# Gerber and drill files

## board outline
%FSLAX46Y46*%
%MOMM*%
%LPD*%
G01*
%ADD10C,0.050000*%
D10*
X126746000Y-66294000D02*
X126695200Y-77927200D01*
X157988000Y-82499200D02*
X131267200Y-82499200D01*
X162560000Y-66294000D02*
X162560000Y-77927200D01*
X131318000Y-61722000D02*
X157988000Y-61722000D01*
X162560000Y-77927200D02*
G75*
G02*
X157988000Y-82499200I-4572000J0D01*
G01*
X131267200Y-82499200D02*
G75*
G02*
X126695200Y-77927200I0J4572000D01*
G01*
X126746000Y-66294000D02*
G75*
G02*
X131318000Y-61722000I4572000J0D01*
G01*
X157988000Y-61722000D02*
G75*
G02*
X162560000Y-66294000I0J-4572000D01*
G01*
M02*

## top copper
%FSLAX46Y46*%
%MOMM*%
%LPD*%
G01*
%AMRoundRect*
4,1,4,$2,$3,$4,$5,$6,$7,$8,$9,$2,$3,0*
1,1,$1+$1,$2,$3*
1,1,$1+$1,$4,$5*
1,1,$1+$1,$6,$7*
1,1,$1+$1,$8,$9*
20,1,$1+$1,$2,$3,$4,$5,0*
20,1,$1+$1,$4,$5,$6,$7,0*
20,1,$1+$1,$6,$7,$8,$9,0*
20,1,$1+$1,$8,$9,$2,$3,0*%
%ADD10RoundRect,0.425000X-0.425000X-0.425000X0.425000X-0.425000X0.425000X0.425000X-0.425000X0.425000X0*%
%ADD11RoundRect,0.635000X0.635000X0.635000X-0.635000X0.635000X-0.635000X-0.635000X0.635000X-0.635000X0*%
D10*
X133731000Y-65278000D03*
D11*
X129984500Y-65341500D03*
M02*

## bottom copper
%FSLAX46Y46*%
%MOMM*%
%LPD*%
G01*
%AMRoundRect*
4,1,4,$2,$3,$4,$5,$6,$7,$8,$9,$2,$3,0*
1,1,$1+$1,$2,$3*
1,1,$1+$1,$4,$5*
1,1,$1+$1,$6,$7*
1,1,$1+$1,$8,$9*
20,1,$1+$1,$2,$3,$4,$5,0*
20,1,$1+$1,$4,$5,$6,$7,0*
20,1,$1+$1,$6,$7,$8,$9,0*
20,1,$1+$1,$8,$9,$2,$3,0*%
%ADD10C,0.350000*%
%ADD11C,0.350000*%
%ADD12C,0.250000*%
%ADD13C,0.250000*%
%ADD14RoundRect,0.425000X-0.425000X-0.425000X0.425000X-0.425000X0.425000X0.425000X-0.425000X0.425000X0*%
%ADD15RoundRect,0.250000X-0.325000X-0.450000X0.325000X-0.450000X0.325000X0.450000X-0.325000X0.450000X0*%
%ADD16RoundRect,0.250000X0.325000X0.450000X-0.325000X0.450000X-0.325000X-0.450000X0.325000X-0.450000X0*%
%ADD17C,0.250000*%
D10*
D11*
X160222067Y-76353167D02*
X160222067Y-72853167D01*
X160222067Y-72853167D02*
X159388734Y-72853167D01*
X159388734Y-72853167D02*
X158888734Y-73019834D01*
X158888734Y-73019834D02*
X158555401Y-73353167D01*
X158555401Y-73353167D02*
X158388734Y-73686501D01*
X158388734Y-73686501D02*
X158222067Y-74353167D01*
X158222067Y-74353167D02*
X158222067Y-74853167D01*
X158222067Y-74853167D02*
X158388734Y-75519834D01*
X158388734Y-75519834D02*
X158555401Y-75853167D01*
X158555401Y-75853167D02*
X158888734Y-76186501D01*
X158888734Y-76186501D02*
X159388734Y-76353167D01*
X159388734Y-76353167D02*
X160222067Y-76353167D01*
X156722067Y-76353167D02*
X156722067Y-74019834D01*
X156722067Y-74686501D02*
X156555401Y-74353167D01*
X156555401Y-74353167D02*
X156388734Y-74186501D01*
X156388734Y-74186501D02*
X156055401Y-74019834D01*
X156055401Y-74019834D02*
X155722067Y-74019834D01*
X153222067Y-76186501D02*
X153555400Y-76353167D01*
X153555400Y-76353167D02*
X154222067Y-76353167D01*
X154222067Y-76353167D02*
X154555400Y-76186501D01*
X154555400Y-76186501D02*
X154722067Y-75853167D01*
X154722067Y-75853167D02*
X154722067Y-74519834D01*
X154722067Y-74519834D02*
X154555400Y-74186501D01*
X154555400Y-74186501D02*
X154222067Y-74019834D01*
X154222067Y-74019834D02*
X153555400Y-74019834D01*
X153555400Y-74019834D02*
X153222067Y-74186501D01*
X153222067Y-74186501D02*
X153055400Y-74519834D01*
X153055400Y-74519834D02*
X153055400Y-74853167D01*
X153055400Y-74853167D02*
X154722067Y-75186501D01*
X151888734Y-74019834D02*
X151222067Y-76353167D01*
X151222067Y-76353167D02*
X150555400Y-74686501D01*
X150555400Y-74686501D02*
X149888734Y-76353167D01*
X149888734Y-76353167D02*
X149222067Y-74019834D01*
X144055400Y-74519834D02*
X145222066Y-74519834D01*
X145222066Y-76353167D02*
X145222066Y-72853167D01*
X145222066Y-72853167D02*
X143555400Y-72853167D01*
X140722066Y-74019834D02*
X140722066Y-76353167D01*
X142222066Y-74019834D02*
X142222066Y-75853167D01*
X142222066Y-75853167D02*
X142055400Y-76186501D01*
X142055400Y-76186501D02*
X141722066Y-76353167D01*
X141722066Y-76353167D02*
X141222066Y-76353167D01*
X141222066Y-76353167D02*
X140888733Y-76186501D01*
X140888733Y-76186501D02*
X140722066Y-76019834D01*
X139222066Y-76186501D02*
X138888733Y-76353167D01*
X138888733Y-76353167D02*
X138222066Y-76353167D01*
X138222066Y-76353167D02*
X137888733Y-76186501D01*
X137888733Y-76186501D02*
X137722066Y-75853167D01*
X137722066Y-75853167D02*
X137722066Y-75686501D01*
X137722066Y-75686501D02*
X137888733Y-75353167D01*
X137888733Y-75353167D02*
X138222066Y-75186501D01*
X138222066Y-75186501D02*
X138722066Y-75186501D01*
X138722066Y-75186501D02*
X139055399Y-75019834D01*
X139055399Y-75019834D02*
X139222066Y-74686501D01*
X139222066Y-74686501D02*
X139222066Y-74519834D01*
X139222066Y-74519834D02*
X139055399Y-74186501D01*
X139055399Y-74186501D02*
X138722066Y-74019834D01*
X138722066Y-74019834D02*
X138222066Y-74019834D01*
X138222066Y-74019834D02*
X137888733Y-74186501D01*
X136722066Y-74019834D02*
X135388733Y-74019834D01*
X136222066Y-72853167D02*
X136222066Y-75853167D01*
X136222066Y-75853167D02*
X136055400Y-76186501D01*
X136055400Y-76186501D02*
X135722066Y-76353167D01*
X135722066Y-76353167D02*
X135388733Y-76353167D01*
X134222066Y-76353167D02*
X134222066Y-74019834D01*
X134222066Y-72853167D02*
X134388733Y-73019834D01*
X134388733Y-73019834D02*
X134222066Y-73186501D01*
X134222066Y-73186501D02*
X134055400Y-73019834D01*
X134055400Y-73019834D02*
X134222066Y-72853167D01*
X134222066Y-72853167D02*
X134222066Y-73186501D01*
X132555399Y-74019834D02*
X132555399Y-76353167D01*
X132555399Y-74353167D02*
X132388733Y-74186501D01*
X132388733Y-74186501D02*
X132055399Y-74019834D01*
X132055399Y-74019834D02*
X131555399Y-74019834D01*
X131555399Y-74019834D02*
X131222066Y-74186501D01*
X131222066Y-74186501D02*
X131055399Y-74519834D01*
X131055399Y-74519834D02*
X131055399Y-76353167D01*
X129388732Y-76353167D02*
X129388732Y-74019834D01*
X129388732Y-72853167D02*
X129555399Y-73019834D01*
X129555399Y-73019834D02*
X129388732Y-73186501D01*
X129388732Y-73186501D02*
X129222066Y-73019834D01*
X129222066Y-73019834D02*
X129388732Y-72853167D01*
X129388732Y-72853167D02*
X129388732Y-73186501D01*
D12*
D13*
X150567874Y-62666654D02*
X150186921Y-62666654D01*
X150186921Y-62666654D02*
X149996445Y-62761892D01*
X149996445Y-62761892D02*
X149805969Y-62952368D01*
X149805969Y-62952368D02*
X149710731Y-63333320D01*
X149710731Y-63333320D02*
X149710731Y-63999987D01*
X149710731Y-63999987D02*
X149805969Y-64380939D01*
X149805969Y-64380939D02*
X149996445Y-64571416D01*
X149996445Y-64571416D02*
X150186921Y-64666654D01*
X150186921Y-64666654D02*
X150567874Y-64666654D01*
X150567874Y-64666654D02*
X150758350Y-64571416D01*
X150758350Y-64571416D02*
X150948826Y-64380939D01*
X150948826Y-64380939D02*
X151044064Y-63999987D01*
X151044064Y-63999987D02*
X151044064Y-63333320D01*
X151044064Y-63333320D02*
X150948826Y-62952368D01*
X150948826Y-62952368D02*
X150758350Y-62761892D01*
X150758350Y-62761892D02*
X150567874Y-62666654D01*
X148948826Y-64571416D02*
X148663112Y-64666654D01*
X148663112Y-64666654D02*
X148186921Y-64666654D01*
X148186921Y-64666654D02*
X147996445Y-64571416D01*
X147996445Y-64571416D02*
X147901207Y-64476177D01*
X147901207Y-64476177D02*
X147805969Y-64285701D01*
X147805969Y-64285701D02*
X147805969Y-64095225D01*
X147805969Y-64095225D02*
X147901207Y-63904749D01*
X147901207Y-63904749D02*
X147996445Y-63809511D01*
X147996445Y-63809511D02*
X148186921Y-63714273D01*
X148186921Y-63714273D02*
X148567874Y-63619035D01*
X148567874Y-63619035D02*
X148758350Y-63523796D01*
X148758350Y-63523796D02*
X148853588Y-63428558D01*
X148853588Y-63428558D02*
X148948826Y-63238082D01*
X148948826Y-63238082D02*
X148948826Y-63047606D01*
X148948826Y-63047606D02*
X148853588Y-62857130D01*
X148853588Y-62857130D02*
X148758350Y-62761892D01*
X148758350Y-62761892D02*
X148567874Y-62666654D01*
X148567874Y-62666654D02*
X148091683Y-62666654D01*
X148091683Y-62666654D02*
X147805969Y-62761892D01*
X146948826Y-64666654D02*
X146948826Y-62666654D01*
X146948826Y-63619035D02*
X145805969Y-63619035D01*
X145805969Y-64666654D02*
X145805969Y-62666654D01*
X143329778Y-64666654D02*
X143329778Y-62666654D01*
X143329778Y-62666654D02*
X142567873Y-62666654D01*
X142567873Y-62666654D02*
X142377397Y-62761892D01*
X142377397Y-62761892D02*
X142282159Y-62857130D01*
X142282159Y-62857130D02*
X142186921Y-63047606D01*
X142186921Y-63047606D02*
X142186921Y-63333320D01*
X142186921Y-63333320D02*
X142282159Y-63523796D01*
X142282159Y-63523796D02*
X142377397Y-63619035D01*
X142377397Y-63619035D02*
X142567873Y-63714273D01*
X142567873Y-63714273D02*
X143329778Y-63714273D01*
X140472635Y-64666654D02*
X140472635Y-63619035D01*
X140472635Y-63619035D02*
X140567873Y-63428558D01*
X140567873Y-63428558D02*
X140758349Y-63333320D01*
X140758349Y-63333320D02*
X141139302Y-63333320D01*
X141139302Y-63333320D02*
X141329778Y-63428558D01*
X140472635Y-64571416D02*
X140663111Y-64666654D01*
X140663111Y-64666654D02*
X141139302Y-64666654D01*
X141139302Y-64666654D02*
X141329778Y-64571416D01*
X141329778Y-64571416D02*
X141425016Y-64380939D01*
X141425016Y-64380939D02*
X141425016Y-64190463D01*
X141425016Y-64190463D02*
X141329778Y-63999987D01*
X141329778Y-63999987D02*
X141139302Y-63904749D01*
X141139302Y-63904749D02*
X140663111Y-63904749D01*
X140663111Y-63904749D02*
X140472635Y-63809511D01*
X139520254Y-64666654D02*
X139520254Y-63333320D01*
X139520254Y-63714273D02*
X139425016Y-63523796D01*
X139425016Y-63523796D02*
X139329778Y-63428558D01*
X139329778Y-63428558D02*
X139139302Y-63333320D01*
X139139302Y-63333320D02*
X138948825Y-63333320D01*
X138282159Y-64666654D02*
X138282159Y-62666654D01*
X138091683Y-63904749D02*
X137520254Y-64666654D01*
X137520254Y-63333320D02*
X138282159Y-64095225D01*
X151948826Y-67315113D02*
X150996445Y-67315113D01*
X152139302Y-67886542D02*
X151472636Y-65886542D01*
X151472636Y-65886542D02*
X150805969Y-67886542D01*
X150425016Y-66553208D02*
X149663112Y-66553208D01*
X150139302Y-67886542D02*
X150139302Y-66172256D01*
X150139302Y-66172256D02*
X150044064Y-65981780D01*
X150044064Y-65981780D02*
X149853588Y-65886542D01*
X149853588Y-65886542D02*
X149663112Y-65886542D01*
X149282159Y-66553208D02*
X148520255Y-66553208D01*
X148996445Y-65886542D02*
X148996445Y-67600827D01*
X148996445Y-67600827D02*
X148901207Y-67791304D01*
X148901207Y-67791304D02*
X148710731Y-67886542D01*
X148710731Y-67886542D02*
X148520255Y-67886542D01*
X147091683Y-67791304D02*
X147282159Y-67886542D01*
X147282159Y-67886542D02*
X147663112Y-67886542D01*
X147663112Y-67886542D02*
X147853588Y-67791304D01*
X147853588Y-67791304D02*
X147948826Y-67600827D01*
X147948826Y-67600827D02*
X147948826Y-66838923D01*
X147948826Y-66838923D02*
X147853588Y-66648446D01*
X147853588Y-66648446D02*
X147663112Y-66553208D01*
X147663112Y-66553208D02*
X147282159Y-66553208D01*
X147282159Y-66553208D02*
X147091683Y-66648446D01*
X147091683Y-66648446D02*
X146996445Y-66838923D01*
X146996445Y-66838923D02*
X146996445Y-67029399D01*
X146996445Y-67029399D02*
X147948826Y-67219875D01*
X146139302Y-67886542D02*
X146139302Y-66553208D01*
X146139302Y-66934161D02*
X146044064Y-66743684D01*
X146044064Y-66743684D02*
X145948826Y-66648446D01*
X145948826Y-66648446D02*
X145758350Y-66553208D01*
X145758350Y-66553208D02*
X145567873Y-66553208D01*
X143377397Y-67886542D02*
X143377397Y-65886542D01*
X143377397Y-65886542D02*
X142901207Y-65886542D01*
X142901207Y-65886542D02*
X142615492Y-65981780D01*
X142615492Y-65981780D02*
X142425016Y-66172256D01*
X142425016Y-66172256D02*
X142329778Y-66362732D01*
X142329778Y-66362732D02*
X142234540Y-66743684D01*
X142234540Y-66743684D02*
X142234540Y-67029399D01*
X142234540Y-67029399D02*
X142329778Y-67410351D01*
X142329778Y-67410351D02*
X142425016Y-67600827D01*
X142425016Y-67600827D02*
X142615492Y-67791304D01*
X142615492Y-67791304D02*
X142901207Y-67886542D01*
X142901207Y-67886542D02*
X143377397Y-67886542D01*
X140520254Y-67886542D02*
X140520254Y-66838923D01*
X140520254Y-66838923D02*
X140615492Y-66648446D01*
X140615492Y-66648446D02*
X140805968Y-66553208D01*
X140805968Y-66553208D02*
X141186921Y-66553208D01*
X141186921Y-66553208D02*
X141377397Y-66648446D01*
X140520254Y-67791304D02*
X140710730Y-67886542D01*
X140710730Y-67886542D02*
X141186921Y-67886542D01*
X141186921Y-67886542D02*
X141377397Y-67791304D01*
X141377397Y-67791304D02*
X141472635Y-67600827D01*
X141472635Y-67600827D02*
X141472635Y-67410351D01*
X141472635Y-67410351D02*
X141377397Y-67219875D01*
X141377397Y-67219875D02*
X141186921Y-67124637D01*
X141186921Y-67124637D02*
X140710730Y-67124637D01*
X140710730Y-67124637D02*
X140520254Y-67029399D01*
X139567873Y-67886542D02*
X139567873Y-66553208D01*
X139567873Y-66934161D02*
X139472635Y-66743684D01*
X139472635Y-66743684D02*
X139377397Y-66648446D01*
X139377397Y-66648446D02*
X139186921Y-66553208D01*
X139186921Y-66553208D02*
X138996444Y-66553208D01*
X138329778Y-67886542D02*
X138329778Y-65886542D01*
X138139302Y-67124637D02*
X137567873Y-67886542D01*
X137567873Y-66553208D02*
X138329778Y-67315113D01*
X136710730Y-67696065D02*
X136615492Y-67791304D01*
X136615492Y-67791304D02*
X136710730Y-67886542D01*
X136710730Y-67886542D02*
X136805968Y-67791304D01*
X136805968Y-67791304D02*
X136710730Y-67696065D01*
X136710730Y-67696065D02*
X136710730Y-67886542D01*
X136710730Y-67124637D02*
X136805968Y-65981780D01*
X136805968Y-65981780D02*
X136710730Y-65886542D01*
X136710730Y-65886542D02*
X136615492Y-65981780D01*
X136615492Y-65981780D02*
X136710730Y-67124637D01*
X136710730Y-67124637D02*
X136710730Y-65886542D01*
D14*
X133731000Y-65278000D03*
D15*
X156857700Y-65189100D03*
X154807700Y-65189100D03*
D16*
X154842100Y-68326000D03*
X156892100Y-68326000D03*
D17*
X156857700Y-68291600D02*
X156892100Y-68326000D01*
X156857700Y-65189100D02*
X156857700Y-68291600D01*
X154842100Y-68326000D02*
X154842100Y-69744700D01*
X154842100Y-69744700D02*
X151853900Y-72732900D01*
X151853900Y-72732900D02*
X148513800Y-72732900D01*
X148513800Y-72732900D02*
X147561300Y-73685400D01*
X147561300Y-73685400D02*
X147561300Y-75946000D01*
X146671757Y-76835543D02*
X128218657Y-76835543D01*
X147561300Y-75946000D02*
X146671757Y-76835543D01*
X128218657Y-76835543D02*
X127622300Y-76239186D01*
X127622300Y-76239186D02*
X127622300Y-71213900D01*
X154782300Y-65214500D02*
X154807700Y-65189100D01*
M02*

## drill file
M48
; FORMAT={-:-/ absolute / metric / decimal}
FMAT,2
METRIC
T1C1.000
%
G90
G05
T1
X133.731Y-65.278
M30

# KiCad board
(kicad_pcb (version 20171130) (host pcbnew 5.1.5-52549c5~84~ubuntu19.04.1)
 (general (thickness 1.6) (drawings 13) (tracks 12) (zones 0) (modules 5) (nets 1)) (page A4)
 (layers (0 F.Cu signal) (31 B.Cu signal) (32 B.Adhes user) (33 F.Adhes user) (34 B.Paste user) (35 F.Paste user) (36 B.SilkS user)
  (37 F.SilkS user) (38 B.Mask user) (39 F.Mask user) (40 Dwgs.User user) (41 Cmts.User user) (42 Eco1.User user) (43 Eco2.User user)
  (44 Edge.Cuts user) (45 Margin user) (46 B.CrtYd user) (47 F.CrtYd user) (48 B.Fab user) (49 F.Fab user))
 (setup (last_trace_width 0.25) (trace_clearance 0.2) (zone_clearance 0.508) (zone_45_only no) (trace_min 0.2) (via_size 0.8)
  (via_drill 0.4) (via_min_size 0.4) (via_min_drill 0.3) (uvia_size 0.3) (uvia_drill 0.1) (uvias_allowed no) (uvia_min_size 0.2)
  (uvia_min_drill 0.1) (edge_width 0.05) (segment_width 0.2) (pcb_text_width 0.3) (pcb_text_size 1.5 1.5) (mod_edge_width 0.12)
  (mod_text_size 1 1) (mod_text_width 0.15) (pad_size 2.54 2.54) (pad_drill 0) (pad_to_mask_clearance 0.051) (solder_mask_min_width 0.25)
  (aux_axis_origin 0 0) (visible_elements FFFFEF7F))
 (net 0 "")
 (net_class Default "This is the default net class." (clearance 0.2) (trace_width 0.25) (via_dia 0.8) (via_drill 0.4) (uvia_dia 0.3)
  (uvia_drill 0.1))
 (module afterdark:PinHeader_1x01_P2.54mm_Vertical (layer F.Cu) (at 133.731 65.278)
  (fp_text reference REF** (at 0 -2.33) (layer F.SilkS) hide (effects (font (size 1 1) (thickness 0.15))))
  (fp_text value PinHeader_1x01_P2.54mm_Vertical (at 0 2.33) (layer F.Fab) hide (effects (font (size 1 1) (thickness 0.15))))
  (pad 1 thru_hole roundrect (at 0 0) (size 1.7 1.7) (drill 1) (layers *.Cu *.Mask) (roundrect_rratio 0.25)))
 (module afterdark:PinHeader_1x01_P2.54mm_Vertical (layer F.Cu) (at 129.9845 65.3415 180)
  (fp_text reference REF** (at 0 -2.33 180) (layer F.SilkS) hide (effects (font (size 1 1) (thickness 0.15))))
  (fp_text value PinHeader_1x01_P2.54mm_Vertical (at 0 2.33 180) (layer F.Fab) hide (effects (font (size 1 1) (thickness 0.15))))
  (pad 1 smd roundrect (at 0 0 180) (size 2.54 2.54) (layers F.Cu F.Paste F.Mask) (roundrect_rratio 0.25)))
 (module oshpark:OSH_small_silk (layer F.Cu) (at 144.4244 71.8312)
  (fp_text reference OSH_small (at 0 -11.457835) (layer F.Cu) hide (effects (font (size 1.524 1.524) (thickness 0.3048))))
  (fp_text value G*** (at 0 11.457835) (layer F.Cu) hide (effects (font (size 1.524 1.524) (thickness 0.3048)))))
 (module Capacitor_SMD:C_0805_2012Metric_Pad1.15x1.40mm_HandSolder (layer B.Cu) (at 155.8327 65.1891)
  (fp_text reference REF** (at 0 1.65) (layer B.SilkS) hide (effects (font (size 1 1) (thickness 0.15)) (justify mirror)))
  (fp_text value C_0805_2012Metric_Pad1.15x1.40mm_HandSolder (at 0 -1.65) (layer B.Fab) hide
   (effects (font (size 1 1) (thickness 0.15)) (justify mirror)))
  (pad 2 smd roundrect (at 1.025 0) (size 1.15 1.4) (layers B.Cu B.Paste B.Mask) (roundrect_rratio 0.217391))
  (pad 1 smd roundrect (at -1.025 0) (size 1.15 1.4) (layers B.Cu B.Paste B.Mask) (roundrect_rratio 0.217391)))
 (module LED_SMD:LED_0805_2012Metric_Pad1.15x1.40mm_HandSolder (layer B.Cu) (at 155.8671 68.326 180)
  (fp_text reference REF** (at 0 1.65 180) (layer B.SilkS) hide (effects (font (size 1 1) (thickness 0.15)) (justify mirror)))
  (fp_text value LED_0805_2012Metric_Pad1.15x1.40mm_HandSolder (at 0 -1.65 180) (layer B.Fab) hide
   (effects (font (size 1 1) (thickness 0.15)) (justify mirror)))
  (pad 2 smd roundrect (at 1.025 0 180) (size 1.15 1.4) (layers B.Cu B.Paste B.Mask) (roundrect_rratio 0.217391))
  (pad 1 smd roundrect (at -1.025 0 180) (size 1.15 1.4) (layers B.Cu B.Paste B.Mask) (roundrect_rratio 0.217391)))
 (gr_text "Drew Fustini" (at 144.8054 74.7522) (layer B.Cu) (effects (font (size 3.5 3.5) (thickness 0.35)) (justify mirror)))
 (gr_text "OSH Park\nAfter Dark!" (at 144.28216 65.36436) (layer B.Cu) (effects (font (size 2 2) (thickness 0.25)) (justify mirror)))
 (gr_line (start 126.746 66.294) (end 126.6952 77.9272) (layer Edge.Cuts) (width 0.05))
 (gr_line (start 157.988 82.4992) (end 131.2672 82.4992) (layer Edge.Cuts) (width 0.05))
 (gr_line (start 162.56 66.294) (end 162.56 77.9272) (layer Edge.Cuts) (width 0.05))
 (gr_line (start 131.318 61.722) (end 157.988 61.722) (layer Edge.Cuts) (width 0.05))
 (gr_arc (start 157.988 77.9272) (end 157.988 82.4992) (angle -90) (layer Edge.Cuts) (width 0.05))
 (gr_arc (start 131.2672 77.9272) (end 126.6952 77.9272) (angle -90) (layer Edge.Cuts) (width 0.05))
 (gr_arc (start 131.318 66.294) (end 131.318 61.722) (angle -90) (layer Edge.Cuts) (width 0.05))
 (gr_arc (start 157.988 66.294) (end 162.56 66.294) (angle -90) (layer Edge.Cuts) (width 0.05))
 (segment (start 156.8577 68.2916) (end 156.8921 68.326) (width 0.25) (layer B.Cu) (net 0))
 (segment (start 156.8577 65.1891) (end 156.8577 68.2916) (width 0.25) (layer B.Cu) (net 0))
 (segment (start 154.8421 68.326) (end 154.8421 69.7447) (width 0.25) (layer B.Cu) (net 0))
 (segment (start 154.8421 69.7447) (end 151.8539 72.7329) (width 0.25) (layer B.Cu) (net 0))
 (segment (start 151.8539 72.7329) (end 148.5138 72.7329) (width 0.25) (layer B.Cu) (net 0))
 (segment (start 148.5138 72.7329) (end 147.5613 73.6854) (width 0.25) (layer B.Cu) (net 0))
 (segment (start 147.5613 73.6854) (end 147.5613 75.946) (width 0.25) (layer B.Cu) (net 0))
 (segment (start 146.671757 76.835543) (end 128.218657 76.835543) (width 0.25) (layer B.Cu) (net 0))
 (segment (start 147.5613 75.946) (end 146.671757 76.835543) (width 0.25) (layer B.Cu) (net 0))
 (segment (start 128.218657 76.835543) (end 127.6223 76.239186) (width 0.25) (layer B.Cu) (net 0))
 (segment (start 127.6223 76.239186) (end 127.6223 71.2139) (width 0.25) (layer B.Cu) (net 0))
 (segment (start 154.7823 65.2145) (end 154.8077 65.1891) (width 0.25) (layer B.Cu) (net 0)))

